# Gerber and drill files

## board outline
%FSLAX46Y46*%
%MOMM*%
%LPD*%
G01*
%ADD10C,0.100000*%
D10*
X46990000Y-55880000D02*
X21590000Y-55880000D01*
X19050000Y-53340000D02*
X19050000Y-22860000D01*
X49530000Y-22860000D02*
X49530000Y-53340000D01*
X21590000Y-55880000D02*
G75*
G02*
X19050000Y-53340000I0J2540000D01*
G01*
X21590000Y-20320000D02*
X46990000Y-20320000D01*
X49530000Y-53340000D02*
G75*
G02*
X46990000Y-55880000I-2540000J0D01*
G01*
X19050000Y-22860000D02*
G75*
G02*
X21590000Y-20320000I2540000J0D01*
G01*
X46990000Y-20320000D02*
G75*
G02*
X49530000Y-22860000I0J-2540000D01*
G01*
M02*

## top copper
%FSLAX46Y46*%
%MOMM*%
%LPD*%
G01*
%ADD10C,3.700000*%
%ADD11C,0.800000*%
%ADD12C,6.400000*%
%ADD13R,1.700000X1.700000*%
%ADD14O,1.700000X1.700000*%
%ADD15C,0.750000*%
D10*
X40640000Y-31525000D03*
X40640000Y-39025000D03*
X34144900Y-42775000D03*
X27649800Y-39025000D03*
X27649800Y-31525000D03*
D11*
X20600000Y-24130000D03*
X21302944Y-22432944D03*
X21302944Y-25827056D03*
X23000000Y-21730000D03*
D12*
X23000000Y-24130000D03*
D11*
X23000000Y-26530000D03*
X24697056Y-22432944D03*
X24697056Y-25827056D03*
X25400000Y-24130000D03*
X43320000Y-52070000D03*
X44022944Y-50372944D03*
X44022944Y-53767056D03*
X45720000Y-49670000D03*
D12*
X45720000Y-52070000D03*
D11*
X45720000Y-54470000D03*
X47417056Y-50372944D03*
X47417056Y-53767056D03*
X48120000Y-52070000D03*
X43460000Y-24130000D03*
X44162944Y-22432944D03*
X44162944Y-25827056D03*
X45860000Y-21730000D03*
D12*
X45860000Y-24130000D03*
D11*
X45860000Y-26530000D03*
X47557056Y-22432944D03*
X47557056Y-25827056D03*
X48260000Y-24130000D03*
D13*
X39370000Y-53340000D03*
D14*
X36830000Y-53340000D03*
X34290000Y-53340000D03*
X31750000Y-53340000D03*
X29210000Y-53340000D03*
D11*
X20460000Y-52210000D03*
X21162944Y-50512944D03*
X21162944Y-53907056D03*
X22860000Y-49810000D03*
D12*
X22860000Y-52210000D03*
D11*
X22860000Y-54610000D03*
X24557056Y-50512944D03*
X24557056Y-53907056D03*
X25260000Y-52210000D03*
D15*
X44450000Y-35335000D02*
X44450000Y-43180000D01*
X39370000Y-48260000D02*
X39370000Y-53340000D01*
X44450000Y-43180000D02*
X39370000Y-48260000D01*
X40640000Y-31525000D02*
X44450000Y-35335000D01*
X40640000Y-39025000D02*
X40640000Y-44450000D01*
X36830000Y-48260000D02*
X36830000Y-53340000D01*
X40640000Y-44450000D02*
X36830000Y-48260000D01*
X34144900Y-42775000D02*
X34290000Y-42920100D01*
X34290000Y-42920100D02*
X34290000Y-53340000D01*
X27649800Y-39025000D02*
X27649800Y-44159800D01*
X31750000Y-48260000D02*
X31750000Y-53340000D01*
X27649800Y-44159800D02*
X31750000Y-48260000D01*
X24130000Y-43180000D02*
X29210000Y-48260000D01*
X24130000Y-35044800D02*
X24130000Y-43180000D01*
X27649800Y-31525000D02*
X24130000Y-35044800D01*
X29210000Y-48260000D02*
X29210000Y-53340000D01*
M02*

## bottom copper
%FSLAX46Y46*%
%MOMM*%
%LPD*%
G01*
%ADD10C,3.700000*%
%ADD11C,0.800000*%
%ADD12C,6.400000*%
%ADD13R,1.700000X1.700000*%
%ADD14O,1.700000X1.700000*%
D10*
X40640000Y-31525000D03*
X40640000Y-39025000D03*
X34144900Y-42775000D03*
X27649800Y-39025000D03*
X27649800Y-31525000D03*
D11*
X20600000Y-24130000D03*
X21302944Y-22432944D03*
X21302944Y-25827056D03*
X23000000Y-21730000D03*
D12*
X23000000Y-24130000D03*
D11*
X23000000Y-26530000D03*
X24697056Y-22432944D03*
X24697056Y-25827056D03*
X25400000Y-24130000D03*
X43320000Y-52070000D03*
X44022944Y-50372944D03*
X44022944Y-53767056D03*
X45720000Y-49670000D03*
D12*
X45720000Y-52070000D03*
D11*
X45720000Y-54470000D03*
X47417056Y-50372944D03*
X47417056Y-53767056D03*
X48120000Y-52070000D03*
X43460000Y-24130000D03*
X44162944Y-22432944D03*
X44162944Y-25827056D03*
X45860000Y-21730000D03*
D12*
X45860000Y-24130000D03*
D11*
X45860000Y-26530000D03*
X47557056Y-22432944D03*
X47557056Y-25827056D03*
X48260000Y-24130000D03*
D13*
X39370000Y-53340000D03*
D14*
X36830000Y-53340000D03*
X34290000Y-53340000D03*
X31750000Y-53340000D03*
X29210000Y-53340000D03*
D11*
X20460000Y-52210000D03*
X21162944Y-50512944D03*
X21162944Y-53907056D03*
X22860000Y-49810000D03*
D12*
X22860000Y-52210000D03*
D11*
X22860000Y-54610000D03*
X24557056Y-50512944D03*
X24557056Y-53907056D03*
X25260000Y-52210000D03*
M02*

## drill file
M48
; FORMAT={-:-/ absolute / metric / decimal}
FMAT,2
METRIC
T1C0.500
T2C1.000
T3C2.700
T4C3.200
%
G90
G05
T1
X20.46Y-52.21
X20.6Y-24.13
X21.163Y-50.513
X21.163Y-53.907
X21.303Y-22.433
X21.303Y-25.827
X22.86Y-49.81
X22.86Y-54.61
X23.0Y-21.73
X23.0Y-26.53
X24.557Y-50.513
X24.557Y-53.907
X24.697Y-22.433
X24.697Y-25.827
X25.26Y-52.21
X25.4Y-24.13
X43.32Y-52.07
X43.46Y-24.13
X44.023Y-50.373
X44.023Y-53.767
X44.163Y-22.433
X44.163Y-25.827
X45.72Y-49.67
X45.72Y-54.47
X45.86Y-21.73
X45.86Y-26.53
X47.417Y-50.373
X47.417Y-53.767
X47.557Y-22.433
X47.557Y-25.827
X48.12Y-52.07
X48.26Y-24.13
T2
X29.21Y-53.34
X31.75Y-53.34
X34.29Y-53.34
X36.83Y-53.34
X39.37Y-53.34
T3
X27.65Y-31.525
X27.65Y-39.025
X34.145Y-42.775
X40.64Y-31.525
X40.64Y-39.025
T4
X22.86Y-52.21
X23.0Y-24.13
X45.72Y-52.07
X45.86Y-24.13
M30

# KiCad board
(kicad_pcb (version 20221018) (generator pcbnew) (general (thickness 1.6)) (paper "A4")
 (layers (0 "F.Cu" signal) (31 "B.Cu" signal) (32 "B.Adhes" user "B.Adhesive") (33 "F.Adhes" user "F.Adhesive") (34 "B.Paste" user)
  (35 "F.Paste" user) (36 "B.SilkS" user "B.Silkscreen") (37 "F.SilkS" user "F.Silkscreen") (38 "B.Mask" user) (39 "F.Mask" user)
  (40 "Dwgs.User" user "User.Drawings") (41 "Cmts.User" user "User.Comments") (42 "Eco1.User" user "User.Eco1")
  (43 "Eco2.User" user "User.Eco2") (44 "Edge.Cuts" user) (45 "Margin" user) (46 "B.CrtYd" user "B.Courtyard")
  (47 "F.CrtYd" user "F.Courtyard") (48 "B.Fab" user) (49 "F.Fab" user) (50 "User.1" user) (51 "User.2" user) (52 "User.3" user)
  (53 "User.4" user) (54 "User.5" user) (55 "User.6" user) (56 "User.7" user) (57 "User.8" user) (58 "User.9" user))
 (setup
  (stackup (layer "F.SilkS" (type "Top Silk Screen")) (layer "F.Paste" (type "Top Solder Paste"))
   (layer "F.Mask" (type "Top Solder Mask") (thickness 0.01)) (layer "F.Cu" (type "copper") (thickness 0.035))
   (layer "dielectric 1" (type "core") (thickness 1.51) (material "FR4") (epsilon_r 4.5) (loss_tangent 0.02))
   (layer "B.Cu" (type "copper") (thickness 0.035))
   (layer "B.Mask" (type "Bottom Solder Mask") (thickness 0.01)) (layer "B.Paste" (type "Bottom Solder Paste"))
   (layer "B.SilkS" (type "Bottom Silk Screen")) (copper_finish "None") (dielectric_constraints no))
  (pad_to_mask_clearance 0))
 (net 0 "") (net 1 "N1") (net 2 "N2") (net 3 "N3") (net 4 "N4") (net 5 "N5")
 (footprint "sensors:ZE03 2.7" (layer "F.Cu") (at 34.1449 35.275)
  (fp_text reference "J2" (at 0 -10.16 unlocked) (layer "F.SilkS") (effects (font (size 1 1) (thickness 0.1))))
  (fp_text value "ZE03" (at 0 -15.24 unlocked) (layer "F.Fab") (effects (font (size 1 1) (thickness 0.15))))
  (pad "1" thru_hole circle (at 6.4951 -3.75) (size 3.7 3.7) (drill 2.7) (layers "*.Cu" "*.Mask") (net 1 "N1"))
  (pad "2" thru_hole circle (at 6.4951 3.75) (size 3.7 3.7) (drill 2.7) (layers "*.Cu" "*.Mask") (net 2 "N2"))
  (pad "3" thru_hole circle (at 0 7.5) (size 3.7 3.7) (drill 2.7) (layers "*.Cu" "*.Mask") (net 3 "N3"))
  (pad "4" thru_hole circle (at -6.4951 3.75) (size 3.7 3.7) (drill 2.7) (layers "*.Cu" "*.Mask") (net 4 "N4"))
  (pad "5" thru_hole circle (at -6.4951 -3.75) (size 3.7 3.7) (drill 2.7) (layers "*.Cu" "*.Mask") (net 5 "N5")))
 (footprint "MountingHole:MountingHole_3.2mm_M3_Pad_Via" (layer "F.Cu") (at 23 24.13)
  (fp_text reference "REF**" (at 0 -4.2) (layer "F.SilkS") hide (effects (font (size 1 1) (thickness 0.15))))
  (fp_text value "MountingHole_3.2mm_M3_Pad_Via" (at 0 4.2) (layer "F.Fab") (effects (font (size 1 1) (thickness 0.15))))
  (pad "1" thru_hole circle (at -2.4 0) (size 0.8 0.8) (drill 0.5) (layers "*.Cu" "*.Mask") (zone_connect 2))
  (pad "1" thru_hole circle (at -1.697056 -1.697056) (size 0.8 0.8) (drill 0.5) (layers "*.Cu" "*.Mask") (zone_connect 2))
  (pad "1" thru_hole circle (at -1.697056 1.697056) (size 0.8 0.8) (drill 0.5) (layers "*.Cu" "*.Mask") (zone_connect 2))
  (pad "1" thru_hole circle (at 0 -2.4) (size 0.8 0.8) (drill 0.5) (layers "*.Cu" "*.Mask") (zone_connect 2))
  (pad "1" thru_hole circle (at 0 0) (size 6.4 6.4) (drill 3.2) (layers "*.Cu" "*.Mask"))
  (pad "1" thru_hole circle (at 0 2.4) (size 0.8 0.8) (drill 0.5) (layers "*.Cu" "*.Mask") (zone_connect 2))
  (pad "1" thru_hole circle (at 1.697056 -1.697056) (size 0.8 0.8) (drill 0.5) (layers "*.Cu" "*.Mask") (zone_connect 2))
  (pad "1" thru_hole circle (at 1.697056 1.697056) (size 0.8 0.8) (drill 0.5) (layers "*.Cu" "*.Mask") (zone_connect 2))
  (pad "1" thru_hole circle (at 2.4 0) (size 0.8 0.8) (drill 0.5) (layers "*.Cu" "*.Mask") (zone_connect 2)))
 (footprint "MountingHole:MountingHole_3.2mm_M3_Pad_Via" (layer "F.Cu") (at 45.72 52.07)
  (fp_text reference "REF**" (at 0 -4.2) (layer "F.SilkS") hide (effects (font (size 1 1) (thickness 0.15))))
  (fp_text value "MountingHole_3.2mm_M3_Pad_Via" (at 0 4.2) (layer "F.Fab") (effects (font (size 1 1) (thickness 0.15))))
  (pad "1" thru_hole circle (at -2.4 0) (size 0.8 0.8) (drill 0.5) (layers "*.Cu" "*.Mask") (zone_connect 2))
  (pad "1" thru_hole circle (at -1.697056 -1.697056) (size 0.8 0.8) (drill 0.5) (layers "*.Cu" "*.Mask") (zone_connect 2))
  (pad "1" thru_hole circle (at -1.697056 1.697056) (size 0.8 0.8) (drill 0.5) (layers "*.Cu" "*.Mask") (zone_connect 2))
  (pad "1" thru_hole circle (at 0 -2.4) (size 0.8 0.8) (drill 0.5) (layers "*.Cu" "*.Mask") (zone_connect 2))
  (pad "1" thru_hole circle (at 0 0) (size 6.4 6.4) (drill 3.2) (layers "*.Cu" "*.Mask"))
  (pad "1" thru_hole circle (at 0 2.4) (size 0.8 0.8) (drill 0.5) (layers "*.Cu" "*.Mask") (zone_connect 2))
  (pad "1" thru_hole circle (at 1.697056 -1.697056) (size 0.8 0.8) (drill 0.5) (layers "*.Cu" "*.Mask") (zone_connect 2))
  (pad "1" thru_hole circle (at 1.697056 1.697056) (size 0.8 0.8) (drill 0.5) (layers "*.Cu" "*.Mask") (zone_connect 2))
  (pad "1" thru_hole circle (at 2.4 0) (size 0.8 0.8) (drill 0.5) (layers "*.Cu" "*.Mask") (zone_connect 2)))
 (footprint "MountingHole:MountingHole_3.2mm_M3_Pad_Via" (layer "F.Cu") (at 45.86 24.13)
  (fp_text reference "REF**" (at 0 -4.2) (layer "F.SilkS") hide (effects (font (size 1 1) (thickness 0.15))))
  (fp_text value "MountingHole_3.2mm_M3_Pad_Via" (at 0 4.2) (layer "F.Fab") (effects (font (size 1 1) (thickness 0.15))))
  (pad "1" thru_hole circle (at -2.4 0) (size 0.8 0.8) (drill 0.5) (layers "*.Cu" "*.Mask") (zone_connect 2))
  (pad "1" thru_hole circle (at -1.697056 -1.697056) (size 0.8 0.8) (drill 0.5) (layers "*.Cu" "*.Mask") (zone_connect 2))
  (pad "1" thru_hole circle (at -1.697056 1.697056) (size 0.8 0.8) (drill 0.5) (layers "*.Cu" "*.Mask") (zone_connect 2))
  (pad "1" thru_hole circle (at 0 -2.4) (size 0.8 0.8) (drill 0.5) (layers "*.Cu" "*.Mask") (zone_connect 2))
  (pad "1" thru_hole circle (at 0 0) (size 6.4 6.4) (drill 3.2) (layers "*.Cu" "*.Mask"))
  (pad "1" thru_hole circle (at 0 2.4) (size 0.8 0.8) (drill 0.5) (layers "*.Cu" "*.Mask") (zone_connect 2))
  (pad "1" thru_hole circle (at 1.697056 -1.697056) (size 0.8 0.8) (drill 0.5) (layers "*.Cu" "*.Mask") (zone_connect 2))
  (pad "1" thru_hole circle (at 1.697056 1.697056) (size 0.8 0.8) (drill 0.5) (layers "*.Cu" "*.Mask") (zone_connect 2))
  (pad "1" thru_hole circle (at 2.4 0) (size 0.8 0.8) (drill 0.5) (layers "*.Cu" "*.Mask") (zone_connect 2)))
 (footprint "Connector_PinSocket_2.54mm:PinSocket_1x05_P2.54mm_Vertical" (layer "F.Cu") (at 39.37 53.34 -90)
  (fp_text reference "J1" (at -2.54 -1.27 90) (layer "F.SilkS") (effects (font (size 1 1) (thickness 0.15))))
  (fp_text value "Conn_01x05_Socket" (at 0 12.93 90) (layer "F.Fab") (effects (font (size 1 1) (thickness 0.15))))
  (pad "1" thru_hole rect (at 0 0 270) (size 1.7 1.7) (drill 1) (layers "*.Cu" "*.Mask") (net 1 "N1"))
  (pad "2" thru_hole oval (at 0 2.54 270) (size 1.7 1.7) (drill 1) (layers "*.Cu" "*.Mask") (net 2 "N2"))
  (pad "3" thru_hole oval (at 0 5.08 270) (size 1.7 1.7) (drill 1) (layers "*.Cu" "*.Mask") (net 3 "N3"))
  (pad "4" thru_hole oval (at 0 7.62 270) (size 1.7 1.7) (drill 1) (layers "*.Cu" "*.Mask") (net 4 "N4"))
  (pad "5" thru_hole oval (at 0 10.16 270) (size 1.7 1.7) (drill 1) (layers "*.Cu" "*.Mask") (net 5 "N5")))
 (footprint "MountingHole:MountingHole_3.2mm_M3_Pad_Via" (layer "F.Cu") (at 22.86 52.21)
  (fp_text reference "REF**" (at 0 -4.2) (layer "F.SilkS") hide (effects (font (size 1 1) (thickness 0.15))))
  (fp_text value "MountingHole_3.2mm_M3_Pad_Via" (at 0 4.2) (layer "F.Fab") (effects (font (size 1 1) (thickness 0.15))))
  (pad "1" thru_hole circle (at -2.4 0) (size 0.8 0.8) (drill 0.5) (layers "*.Cu" "*.Mask") (zone_connect 2))
  (pad "1" thru_hole circle (at -1.697056 -1.697056) (size 0.8 0.8) (drill 0.5) (layers "*.Cu" "*.Mask") (zone_connect 2))
  (pad "1" thru_hole circle (at -1.697056 1.697056) (size 0.8 0.8) (drill 0.5) (layers "*.Cu" "*.Mask") (zone_connect 2))
  (pad "1" thru_hole circle (at 0 -2.4) (size 0.8 0.8) (drill 0.5) (layers "*.Cu" "*.Mask") (zone_connect 2))
  (pad "1" thru_hole circle (at 0 0) (size 6.4 6.4) (drill 3.2) (layers "*.Cu" "*.Mask"))
  (pad "1" thru_hole circle (at 0 2.4) (size 0.8 0.8) (drill 0.5) (layers "*.Cu" "*.Mask") (zone_connect 2))
  (pad "1" thru_hole circle (at 1.697056 -1.697056) (size 0.8 0.8) (drill 0.5) (layers "*.Cu" "*.Mask") (zone_connect 2))
  (pad "1" thru_hole circle (at 1.697056 1.697056) (size 0.8 0.8) (drill 0.5) (layers "*.Cu" "*.Mask") (zone_connect 2))
  (pad "1" thru_hole circle (at 2.4 0) (size 0.8 0.8) (drill 0.5) (layers "*.Cu" "*.Mask") (zone_connect 2)))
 (gr_line (start 46.99 55.88) (end 21.59 55.88) (stroke (width 0.1) (type default)) (layer "Edge.Cuts"))
 (gr_line (start 19.05 53.34) (end 19.05 22.86) (stroke (width 0.1) (type default)) (layer "Edge.Cuts"))
 (gr_line (start 49.53 22.86) (end 49.53 53.34) (stroke (width 0.1) (type default)) (layer "Edge.Cuts"))
 (gr_arc (start 21.59 55.88) (mid 19.793949 55.136051) (end 19.05 53.34) (stroke (width 0.1) (type default)) (layer "Edge.Cuts"))
 (gr_line (start 21.59 20.32) (end 46.99 20.32) (stroke (width 0.1) (type default)) (layer "Edge.Cuts"))
 (gr_arc (start 49.53 53.34) (mid 48.786051 55.136051) (end 46.99 55.88) (stroke (width 0.1) (type default)) (layer "Edge.Cuts"))
 (gr_arc (start 19.05 22.86) (mid 19.793949 21.063949) (end 21.59 20.32) (stroke (width 0.1) (type default)) (layer "Edge.Cuts"))
 (gr_arc (start 46.99 20.32) (mid 48.786051 21.063949) (end 49.53 22.86) (stroke (width 0.1) (type default)) (layer "Edge.Cuts"))
 (segment (start 44.45 35.335) (end 44.45 43.18) (width 0.75) (layer "F.Cu") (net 1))
 (segment (start 39.37 48.26) (end 39.37 53.34) (width 0.75) (layer "F.Cu") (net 1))
 (segment (start 44.45 43.18) (end 39.37 48.26) (width 0.75) (layer "F.Cu") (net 1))
 (segment (start 40.64 31.525) (end 44.45 35.335) (width 0.75) (layer "F.Cu") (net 1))
 (segment (start 40.64 39.025) (end 40.64 44.45) (width 0.75) (layer "F.Cu") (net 2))
 (segment (start 36.83 48.26) (end 36.83 53.34) (width 0.75) (layer "F.Cu") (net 2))
 (segment (start 40.64 44.45) (end 36.83 48.26) (width 0.75) (layer "F.Cu") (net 2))
 (segment (start 34.1449 42.775) (end 34.29 42.9201) (width 0.75) (layer "F.Cu") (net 3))
 (segment (start 34.29 42.9201) (end 34.29 53.34) (width 0.75) (layer "F.Cu") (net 3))
 (segment (start 27.6498 39.025) (end 27.6498 44.1598) (width 0.75) (layer "F.Cu") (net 4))
 (segment (start 31.75 48.26) (end 31.75 53.34) (width 0.75) (layer "F.Cu") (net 4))
 (segment (start 27.6498 44.1598) (end 31.75 48.26) (width 0.75) (layer "F.Cu") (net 4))
 (segment (start 24.13 43.18) (end 29.21 48.26) (width 0.75) (layer "F.Cu") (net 5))
 (segment (start 24.13 35.0448) (end 24.13 43.18) (width 0.75) (layer "F.Cu") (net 5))
 (segment (start 27.6498 31.525) (end 24.13 35.0448) (width 0.75) (layer "F.Cu") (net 5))
 (segment (start 29.21 48.26) (end 29.21 53.34) (width 0.75) (layer "F.Cu") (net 5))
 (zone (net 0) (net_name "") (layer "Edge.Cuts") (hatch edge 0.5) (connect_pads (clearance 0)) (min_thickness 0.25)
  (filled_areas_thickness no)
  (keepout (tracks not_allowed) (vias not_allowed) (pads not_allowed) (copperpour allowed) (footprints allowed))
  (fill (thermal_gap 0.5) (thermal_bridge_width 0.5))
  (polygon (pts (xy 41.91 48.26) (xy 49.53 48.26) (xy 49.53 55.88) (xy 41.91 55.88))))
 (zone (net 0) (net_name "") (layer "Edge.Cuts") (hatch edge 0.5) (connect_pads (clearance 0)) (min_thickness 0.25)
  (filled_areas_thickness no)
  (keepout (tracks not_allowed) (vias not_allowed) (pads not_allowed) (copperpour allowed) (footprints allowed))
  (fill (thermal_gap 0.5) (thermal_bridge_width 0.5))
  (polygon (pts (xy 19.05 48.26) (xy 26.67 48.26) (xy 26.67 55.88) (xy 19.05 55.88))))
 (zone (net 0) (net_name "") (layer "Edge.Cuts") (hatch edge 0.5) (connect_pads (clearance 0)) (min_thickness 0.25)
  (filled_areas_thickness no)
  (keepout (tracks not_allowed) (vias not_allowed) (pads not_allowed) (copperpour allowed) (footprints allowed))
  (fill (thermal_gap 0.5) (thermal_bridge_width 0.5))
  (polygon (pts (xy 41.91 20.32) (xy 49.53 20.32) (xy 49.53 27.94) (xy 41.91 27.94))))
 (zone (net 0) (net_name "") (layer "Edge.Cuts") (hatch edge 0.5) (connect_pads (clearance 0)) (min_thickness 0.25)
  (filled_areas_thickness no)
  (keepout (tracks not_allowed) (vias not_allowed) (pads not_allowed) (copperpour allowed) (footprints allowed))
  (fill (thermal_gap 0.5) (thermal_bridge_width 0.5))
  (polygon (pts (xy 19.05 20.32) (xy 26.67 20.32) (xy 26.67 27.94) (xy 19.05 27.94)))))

